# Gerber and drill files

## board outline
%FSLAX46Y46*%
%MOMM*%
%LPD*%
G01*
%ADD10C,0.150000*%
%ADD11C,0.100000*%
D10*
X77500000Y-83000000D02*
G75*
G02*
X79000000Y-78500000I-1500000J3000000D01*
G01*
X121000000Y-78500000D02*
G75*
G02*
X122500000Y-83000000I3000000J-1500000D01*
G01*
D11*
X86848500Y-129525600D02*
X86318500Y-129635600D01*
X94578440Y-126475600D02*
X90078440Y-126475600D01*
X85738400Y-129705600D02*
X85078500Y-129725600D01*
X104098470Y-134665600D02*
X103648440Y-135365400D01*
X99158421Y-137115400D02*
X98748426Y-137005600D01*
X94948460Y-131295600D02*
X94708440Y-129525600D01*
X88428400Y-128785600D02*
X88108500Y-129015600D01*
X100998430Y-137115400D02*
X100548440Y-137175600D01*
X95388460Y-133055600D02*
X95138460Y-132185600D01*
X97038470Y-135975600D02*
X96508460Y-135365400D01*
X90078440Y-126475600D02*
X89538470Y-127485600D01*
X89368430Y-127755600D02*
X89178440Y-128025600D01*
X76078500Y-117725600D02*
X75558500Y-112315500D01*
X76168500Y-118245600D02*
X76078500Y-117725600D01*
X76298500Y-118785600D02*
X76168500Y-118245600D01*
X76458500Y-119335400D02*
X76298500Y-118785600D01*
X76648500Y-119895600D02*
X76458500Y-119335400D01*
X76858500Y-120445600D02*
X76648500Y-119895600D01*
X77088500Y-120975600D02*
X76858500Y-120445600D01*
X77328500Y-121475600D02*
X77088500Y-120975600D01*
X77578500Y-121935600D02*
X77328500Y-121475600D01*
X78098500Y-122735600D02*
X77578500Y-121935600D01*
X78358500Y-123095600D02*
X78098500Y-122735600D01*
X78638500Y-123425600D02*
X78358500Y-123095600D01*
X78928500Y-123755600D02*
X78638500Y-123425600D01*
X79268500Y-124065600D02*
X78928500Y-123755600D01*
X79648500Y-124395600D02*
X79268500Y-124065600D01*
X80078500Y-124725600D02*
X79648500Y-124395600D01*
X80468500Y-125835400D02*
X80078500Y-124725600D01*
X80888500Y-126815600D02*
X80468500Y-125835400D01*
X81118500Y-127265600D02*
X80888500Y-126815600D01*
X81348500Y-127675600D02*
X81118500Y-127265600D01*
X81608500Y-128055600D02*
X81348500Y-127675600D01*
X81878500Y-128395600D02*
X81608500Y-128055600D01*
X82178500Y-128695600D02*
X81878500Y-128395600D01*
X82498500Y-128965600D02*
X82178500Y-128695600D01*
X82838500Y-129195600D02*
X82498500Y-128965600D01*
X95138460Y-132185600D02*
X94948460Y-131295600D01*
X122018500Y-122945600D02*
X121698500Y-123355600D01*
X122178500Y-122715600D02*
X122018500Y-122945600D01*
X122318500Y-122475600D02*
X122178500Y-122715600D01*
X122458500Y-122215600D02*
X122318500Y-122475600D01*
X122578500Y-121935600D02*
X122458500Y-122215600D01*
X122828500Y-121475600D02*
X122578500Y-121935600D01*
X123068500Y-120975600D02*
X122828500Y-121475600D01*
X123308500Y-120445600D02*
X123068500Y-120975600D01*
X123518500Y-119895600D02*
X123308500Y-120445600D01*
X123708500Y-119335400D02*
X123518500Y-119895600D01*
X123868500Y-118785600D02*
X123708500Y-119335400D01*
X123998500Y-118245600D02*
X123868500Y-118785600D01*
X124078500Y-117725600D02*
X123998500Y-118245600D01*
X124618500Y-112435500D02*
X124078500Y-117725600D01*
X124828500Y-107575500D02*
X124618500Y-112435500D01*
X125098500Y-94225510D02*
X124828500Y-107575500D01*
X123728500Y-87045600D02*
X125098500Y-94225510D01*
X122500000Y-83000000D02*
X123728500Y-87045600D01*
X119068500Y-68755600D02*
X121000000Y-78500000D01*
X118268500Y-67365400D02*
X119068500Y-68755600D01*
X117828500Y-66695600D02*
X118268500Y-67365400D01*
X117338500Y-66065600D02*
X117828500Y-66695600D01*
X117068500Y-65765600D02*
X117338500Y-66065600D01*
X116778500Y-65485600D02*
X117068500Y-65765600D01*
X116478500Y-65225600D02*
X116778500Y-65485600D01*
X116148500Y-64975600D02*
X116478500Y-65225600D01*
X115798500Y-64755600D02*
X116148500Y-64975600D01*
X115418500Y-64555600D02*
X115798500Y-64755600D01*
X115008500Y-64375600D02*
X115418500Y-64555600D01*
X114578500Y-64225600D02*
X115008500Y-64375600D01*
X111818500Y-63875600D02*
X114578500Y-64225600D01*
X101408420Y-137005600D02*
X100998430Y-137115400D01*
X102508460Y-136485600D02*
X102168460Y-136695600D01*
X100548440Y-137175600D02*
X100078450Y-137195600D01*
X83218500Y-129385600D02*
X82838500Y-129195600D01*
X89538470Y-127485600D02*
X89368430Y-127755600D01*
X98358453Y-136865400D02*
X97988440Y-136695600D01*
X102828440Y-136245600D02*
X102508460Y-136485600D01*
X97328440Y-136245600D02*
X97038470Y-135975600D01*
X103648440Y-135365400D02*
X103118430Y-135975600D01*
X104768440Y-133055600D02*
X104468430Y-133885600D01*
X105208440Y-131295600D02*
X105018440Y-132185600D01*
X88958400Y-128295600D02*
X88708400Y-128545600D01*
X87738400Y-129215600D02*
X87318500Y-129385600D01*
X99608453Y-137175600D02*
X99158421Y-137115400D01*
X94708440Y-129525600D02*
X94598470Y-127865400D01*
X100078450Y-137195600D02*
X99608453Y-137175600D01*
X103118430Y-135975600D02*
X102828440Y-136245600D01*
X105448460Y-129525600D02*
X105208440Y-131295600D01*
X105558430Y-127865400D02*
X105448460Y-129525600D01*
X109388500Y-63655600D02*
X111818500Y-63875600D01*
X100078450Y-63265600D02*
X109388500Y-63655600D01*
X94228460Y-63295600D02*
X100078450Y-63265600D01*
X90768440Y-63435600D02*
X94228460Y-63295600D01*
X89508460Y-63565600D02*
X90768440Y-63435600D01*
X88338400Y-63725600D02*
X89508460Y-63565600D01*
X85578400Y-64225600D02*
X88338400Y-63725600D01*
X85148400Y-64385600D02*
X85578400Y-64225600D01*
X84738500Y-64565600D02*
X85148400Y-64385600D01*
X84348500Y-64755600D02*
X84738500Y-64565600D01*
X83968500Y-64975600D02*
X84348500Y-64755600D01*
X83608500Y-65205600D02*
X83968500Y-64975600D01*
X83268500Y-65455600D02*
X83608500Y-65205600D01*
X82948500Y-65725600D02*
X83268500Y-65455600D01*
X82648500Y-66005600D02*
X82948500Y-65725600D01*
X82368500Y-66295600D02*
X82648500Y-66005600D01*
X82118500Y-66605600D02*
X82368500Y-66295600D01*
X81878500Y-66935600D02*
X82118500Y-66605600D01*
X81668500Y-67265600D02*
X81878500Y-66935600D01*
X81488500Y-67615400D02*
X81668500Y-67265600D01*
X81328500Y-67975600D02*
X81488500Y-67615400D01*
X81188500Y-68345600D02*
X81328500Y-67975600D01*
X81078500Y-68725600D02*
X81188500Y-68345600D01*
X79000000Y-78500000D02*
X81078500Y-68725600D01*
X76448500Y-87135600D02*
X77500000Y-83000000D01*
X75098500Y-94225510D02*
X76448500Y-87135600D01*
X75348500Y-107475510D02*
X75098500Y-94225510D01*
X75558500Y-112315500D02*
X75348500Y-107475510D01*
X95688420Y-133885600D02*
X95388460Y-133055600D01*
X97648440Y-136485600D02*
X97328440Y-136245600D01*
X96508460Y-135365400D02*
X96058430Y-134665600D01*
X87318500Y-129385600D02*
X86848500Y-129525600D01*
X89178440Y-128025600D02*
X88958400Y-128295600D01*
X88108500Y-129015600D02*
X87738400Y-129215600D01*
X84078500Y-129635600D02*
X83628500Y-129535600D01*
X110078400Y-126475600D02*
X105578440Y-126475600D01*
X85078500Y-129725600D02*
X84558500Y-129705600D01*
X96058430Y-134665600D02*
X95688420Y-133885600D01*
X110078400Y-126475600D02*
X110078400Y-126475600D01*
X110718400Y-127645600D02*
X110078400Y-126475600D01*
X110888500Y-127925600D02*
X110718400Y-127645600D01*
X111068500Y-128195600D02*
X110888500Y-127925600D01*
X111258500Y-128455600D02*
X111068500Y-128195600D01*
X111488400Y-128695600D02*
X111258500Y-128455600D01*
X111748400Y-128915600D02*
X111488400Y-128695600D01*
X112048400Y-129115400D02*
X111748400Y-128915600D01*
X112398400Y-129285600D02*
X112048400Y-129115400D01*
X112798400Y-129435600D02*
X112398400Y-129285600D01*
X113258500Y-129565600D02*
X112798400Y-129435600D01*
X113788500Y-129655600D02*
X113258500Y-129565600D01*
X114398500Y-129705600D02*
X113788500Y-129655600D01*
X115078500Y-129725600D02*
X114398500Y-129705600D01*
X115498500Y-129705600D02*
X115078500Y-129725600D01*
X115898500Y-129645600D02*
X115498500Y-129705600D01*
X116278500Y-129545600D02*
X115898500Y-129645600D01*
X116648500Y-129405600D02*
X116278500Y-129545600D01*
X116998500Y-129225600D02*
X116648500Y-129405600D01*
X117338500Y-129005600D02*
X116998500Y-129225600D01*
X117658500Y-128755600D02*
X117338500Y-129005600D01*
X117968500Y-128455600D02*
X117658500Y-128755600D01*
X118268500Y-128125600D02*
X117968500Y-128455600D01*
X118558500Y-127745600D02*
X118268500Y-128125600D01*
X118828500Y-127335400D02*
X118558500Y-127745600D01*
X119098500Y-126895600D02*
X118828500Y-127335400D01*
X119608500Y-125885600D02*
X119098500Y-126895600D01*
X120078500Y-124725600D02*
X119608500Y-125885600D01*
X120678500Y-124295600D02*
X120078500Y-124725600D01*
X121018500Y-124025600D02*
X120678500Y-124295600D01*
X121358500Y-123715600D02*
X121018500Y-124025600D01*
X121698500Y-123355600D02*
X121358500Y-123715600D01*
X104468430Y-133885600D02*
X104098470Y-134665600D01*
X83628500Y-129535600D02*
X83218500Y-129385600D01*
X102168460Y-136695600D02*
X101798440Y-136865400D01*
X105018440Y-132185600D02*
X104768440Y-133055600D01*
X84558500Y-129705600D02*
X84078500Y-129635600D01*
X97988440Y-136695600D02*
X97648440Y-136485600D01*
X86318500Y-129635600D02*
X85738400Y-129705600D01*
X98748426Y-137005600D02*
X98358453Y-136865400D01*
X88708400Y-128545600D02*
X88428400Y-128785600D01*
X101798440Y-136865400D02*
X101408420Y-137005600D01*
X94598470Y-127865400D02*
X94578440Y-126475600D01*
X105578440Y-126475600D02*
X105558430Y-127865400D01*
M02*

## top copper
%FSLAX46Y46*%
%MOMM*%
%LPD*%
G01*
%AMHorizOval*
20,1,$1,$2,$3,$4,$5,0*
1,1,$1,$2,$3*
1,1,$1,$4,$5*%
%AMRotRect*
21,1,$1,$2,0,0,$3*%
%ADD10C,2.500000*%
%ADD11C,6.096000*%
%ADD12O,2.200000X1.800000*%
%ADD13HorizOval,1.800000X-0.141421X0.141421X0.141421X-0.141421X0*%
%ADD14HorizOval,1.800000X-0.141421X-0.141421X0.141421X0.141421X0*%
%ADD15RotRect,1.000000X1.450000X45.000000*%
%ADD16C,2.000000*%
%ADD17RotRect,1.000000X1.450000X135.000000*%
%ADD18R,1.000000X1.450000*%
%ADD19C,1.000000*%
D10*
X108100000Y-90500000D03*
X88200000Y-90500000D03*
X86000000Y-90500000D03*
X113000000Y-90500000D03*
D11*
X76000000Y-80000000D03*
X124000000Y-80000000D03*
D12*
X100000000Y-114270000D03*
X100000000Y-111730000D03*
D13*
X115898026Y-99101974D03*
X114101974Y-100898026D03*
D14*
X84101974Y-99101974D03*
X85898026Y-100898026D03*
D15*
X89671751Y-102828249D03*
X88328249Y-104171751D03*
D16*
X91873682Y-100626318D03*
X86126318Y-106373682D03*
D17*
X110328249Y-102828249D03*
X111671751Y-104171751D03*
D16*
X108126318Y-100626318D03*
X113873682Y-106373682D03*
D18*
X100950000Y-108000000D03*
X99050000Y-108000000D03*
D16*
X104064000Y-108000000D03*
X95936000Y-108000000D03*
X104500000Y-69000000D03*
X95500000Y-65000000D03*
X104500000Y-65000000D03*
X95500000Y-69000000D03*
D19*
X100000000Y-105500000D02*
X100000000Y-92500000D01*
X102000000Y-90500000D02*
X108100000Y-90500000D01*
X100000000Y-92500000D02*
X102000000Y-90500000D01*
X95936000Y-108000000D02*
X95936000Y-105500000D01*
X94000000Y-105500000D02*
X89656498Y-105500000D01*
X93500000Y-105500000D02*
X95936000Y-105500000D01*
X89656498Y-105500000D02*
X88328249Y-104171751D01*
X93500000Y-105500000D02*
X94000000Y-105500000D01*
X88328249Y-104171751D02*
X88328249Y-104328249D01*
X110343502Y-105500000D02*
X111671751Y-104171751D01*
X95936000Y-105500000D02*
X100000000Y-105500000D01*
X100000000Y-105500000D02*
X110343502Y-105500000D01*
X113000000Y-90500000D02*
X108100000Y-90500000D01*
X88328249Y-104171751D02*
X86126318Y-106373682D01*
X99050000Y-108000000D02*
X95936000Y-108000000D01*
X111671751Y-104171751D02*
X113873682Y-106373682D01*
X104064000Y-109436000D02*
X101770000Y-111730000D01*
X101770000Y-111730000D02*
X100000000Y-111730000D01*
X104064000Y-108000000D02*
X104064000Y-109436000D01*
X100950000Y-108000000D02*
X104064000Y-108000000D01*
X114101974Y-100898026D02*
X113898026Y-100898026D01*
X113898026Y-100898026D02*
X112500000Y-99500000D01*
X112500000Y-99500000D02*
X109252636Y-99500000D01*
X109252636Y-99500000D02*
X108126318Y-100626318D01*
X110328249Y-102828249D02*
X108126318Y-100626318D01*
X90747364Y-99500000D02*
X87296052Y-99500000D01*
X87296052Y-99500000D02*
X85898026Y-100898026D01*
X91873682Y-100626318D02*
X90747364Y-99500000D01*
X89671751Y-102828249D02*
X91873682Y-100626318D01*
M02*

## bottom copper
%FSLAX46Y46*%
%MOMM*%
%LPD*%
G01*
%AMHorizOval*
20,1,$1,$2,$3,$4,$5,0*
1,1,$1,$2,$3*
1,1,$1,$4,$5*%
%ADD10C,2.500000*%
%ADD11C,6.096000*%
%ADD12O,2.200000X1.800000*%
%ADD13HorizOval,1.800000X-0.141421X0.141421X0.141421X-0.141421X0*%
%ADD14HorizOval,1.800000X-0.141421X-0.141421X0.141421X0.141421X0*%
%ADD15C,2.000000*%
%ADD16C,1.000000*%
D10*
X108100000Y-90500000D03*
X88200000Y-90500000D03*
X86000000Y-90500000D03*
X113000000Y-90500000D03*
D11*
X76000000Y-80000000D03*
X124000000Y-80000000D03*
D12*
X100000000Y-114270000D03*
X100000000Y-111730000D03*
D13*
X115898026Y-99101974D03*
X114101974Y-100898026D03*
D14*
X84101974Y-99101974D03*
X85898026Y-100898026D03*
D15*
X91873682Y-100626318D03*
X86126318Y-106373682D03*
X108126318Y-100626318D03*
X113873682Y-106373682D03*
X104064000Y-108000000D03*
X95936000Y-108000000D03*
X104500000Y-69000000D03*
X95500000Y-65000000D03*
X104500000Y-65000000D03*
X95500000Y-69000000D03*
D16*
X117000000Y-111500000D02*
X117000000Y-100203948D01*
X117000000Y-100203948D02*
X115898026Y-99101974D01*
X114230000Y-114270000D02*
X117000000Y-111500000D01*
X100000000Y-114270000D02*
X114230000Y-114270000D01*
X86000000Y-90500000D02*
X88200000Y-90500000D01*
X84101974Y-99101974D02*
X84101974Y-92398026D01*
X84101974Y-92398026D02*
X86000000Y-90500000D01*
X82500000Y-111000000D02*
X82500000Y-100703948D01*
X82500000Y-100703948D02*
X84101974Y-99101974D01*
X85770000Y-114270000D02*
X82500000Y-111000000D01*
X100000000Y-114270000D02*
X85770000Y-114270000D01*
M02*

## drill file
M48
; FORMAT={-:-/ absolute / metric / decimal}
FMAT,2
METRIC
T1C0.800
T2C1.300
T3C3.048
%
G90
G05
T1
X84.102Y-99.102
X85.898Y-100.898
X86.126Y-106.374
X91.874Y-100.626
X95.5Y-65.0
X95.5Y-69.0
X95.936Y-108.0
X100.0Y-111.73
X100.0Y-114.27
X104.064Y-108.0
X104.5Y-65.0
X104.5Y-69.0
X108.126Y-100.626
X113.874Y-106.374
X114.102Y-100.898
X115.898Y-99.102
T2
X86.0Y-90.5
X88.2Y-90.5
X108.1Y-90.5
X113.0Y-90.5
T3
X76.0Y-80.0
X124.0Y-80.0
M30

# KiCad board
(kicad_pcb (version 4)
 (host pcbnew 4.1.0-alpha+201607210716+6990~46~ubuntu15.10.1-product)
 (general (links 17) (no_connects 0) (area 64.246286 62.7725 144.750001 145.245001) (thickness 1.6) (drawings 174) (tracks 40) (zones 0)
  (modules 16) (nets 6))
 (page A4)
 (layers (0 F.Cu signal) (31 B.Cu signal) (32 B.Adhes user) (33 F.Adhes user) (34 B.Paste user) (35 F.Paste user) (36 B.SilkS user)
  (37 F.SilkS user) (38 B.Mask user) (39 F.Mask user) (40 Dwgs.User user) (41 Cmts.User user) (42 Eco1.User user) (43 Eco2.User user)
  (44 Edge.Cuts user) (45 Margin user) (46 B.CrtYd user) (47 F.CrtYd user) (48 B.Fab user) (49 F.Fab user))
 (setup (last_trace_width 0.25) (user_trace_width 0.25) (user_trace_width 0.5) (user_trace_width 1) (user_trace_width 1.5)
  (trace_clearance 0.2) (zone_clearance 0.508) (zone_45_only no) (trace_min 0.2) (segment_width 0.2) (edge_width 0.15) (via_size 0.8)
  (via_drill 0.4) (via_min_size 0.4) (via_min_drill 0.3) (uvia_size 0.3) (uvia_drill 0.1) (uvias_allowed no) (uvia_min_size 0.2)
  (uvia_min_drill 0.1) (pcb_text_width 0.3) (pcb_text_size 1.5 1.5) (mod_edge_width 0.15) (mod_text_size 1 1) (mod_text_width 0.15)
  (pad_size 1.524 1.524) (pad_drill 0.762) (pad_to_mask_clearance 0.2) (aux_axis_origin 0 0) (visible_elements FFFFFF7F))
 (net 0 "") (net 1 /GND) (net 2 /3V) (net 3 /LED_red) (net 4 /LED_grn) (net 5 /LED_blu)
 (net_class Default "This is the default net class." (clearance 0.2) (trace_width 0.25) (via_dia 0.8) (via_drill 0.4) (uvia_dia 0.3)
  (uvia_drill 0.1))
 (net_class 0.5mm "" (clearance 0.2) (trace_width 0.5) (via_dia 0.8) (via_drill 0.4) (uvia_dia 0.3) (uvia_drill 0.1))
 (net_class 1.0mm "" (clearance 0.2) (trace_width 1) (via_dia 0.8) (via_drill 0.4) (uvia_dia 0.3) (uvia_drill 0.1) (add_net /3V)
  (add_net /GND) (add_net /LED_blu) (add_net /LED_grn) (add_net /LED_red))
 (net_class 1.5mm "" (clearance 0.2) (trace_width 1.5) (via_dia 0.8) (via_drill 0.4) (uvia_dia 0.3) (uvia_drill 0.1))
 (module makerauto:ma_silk (layer F.Cu) (at 67.1 109.6)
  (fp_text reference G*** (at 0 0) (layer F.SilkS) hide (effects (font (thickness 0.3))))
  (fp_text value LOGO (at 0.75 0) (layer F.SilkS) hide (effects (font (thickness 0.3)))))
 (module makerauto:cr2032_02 (layer B.Cu) (at 100 90.5 90)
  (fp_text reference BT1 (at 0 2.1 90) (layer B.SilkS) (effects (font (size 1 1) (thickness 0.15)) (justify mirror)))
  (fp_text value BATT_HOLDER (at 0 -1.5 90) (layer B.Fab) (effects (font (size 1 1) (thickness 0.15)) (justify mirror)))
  (pad 2 thru_hole circle (at 0 8.1 90) (size 2.5 2.5) (drill 1.3) (layers *.Cu *.Mask B.SilkS) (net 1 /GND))
  (pad 1 thru_hole circle (at 0 -11.8 90) (size 2.5 2.5) (drill 1.3) (layers *.Cu *.Mask B.SilkS) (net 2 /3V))
  (pad 1 thru_hole circle (at 0 -14 90) (size 2.5 2.5) (drill 1.3) (layers *.Cu *.Mask B.SilkS) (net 2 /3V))
  (pad 2 thru_hole circle (at 0 13 90) (size 2.5 2.5) (drill 1.3) (layers *.Cu *.Mask B.SilkS) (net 1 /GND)))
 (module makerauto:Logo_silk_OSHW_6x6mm (layer B.Cu) (at 100 123 180)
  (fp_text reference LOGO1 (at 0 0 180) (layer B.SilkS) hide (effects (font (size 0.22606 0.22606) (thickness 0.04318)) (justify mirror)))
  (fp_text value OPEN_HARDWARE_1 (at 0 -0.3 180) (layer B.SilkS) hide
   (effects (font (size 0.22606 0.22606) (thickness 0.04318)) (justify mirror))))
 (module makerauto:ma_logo (layer F.Cu) (at 100 100)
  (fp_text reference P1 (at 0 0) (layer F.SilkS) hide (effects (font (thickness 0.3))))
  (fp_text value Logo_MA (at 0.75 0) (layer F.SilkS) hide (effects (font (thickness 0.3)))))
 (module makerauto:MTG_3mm (layer F.Cu) (at 76 80)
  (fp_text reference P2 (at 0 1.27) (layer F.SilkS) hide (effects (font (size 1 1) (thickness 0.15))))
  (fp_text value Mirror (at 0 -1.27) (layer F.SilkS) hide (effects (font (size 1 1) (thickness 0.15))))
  (pad 1 thru_hole circle (at 0 0) (size 6.096 6.096) (drill 3.048) (layers *.Cu *.Mask F.SilkS)))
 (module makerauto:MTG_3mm (layer F.Cu) (at 124 80)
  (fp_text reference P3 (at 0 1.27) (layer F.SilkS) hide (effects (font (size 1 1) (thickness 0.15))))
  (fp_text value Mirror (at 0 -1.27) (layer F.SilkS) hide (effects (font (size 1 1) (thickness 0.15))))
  (pad 1 thru_hole circle (at 0 0) (size 6.096 6.096) (drill 3.048) (layers *.Cu *.Mask F.SilkS)))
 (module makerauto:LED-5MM (layer F.Cu) (at 100 113 90)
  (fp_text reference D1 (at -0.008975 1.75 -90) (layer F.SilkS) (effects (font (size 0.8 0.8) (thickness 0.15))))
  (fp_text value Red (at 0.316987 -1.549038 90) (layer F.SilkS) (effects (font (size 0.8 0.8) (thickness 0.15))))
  (pad 1 thru_hole oval (at -1.27 0 90) (size 1.8 2.2) (drill 0.8) (layers *.Cu *.Mask F.SilkS) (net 2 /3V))
  (pad 2 thru_hole oval (at 1.27 0 90) (size 1.8 2.2) (drill 0.8) (layers *.Cu *.Mask F.SilkS) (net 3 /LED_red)))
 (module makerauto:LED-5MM (layer F.Cu) (at 115 100 225)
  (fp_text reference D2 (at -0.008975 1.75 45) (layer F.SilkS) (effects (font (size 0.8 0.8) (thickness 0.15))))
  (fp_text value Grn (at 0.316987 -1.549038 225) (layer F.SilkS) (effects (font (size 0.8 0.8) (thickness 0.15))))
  (pad 1 thru_hole oval (at -1.27 0 225) (size 1.8 2.2) (drill 0.8) (layers *.Cu *.Mask F.SilkS) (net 2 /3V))
  (pad 2 thru_hole oval (at 1.27 0 225) (size 1.8 2.2) (drill 0.8) (layers *.Cu *.Mask F.SilkS) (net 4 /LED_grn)))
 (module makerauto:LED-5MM (layer F.Cu) (at 85 100 315)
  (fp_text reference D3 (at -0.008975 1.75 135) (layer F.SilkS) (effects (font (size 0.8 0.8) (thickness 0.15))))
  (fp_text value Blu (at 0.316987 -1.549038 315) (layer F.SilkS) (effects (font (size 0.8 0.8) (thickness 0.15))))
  (pad 1 thru_hole oval (at -1.27 0 315) (size 1.8 2.2) (drill 0.8) (layers *.Cu *.Mask F.SilkS) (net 2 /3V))
  (pad 2 thru_hole oval (at 1.27 0 315) (size 1.8 2.2) (drill 0.8) (layers *.Cu *.Mask F.SilkS) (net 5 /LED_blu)))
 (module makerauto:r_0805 (layer F.Cu) (at 89 103.5 45)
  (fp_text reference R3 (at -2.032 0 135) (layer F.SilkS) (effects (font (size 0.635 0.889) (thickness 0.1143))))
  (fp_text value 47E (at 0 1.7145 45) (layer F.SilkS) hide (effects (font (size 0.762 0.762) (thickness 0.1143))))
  (pad 2 smd rect (at 0.95 0 45) (size 1 1.45) (layers F.Cu F.Paste F.Mask) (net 5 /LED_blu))
  (pad 1 smd rect (at -0.95 0 45) (size 1 1.45) (layers F.Cu F.Paste F.Mask) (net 1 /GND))
  (pad 2 thru_hole circle (at 4.064 0 45) (size 2 2) (drill 0.8) (layers *.Cu *.Mask F.SilkS) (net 5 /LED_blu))
  (pad 1 thru_hole circle (at -4.064 0 45) (size 2 2) (drill 0.8) (layers *.Cu *.Mask F.SilkS) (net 1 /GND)))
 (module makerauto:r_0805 (layer F.Cu) (at 111 103.5 135)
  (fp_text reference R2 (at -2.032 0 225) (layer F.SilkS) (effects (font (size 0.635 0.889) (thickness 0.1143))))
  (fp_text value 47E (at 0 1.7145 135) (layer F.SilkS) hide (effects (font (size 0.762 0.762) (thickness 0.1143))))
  (pad 2 smd rect (at 0.95 0 135) (size 1 1.45) (layers F.Cu F.Paste F.Mask) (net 4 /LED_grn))
  (pad 1 smd rect (at -0.95 0 135) (size 1 1.45) (layers F.Cu F.Paste F.Mask) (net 1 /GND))
  (pad 2 thru_hole circle (at 4.064 0 135) (size 2 2) (drill 0.8) (layers *.Cu *.Mask F.SilkS) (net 4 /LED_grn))
  (pad 1 thru_hole circle (at -4.064 0 135) (size 2 2) (drill 0.8) (layers *.Cu *.Mask F.SilkS) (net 1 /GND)))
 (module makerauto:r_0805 (layer F.Cu) (at 100 108)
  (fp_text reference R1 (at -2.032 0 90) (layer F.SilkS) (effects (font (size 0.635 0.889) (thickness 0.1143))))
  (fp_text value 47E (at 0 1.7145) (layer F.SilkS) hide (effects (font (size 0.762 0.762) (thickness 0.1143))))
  (pad 2 smd rect (at 0.95 0) (size 1 1.45) (layers F.Cu F.Paste F.Mask) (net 3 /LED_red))
  (pad 1 smd rect (at -0.95 0) (size 1 1.45) (layers F.Cu F.Paste F.Mask) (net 1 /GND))
  (pad 2 thru_hole circle (at 4.064 0) (size 2 2) (drill 0.8) (layers *.Cu *.Mask F.SilkS) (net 3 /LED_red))
  (pad 1 thru_hole circle (at -4.064 0) (size 2 2) (drill 0.8) (layers *.Cu *.Mask F.SilkS) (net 1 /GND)))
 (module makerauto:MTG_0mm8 (layer F.Cu) (at 104.5 69)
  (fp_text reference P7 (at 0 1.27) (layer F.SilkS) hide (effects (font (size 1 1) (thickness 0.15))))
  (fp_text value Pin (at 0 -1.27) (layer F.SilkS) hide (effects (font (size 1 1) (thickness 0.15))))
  (pad 1 thru_hole circle (at 0 0) (size 2 2) (drill 0.8) (layers *.Cu *.Mask F.SilkS)))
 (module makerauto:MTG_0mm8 (layer F.Cu) (at 95.5 65)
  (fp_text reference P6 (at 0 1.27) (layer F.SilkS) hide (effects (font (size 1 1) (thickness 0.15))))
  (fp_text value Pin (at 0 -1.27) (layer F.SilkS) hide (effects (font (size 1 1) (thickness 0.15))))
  (pad 1 thru_hole circle (at 0 0) (size 2 2) (drill 0.8) (layers *.Cu *.Mask F.SilkS)))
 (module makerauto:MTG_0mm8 (layer F.Cu) (at 104.5 65)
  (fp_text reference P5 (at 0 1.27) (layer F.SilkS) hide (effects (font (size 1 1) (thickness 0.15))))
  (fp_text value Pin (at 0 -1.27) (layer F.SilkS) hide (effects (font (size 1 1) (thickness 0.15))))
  (pad 1 thru_hole circle (at 0 0) (size 2 2) (drill 0.8) (layers *.Cu *.Mask F.SilkS)))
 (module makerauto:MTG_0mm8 (layer F.Cu) (at 95.5 69)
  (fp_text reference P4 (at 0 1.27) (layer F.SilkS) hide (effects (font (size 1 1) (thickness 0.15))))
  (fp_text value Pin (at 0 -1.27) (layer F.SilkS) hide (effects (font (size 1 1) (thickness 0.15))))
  (pad 1 thru_hole circle (at 0 0) (size 2 2) (drill 0.8) (layers *.Cu *.Mask F.SilkS)))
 (gr_arc (start 76 80) (end 77.5 83) (angle 270) (layer Edge.Cuts) (width 0.15))
 (gr_arc (start 124 80) (end 121 78.5) (angle 270) (layer Edge.Cuts) (width 0.15))
 (gr_line (start 86.8485 129.5256) (end 86.3185 129.6356) (layer Edge.Cuts) (width 0.1))
 (gr_line (start 94.57844 126.4756) (end 90.07844 126.4756) (layer Edge.Cuts) (width 0.1))
 (gr_line (start 85.7384 129.7056) (end 85.0785 129.7256) (layer Edge.Cuts) (width 0.1))
 (gr_line (start 104.09847 134.6656) (end 103.64844 135.3654) (layer Edge.Cuts) (width 0.1))
 (gr_line (start 99.158421 137.1154) (end 98.748426 137.0056) (layer Edge.Cuts) (width 0.1))
 (gr_line (start 94.94846 131.2956) (end 94.70844 129.5256) (layer Edge.Cuts) (width 0.1))
 (gr_line (start 88.4284 128.7856) (end 88.1085 129.0156) (layer Edge.Cuts) (width 0.1))
 (gr_line (start 100.99843 137.1154) (end 100.54844 137.1756) (layer Edge.Cuts) (width 0.1))
 (gr_line (start 95.38846 133.0556) (end 95.13846 132.1856) (layer Edge.Cuts) (width 0.1))
 (gr_line (start 97.03847 135.9756) (end 96.50846 135.3654) (layer Edge.Cuts) (width 0.1))
 (gr_line (start 90.07844 126.4756) (end 89.53847 127.4856) (layer Edge.Cuts) (width 0.1))
 (gr_line (start 89.36843 127.7556) (end 89.17844 128.0256) (layer Edge.Cuts) (width 0.1))
 (gr_line (start 76.0785 117.7256) (end 75.5585 112.3155) (layer Edge.Cuts) (width 0.1))
 (gr_line (start 76.1685 118.2456) (end 76.0785 117.7256) (layer Edge.Cuts) (width 0.1))
 (gr_line (start 76.2985 118.7856) (end 76.1685 118.2456) (layer Edge.Cuts) (width 0.1))
 (gr_line (start 76.4585 119.3354) (end 76.2985 118.7856) (layer Edge.Cuts) (width 0.1))
 (gr_line (start 76.6485 119.8956) (end 76.4585 119.3354) (layer Edge.Cuts) (width 0.1))
 (gr_line (start 76.8585 120.4456) (end 76.6485 119.8956) (layer Edge.Cuts) (width 0.1))
 (gr_line (start 77.0885 120.9756) (end 76.8585 120.4456) (layer Edge.Cuts) (width 0.1))
 (gr_line (start 77.3285 121.4756) (end 77.0885 120.9756) (layer Edge.Cuts) (width 0.1))
 (gr_line (start 77.5785 121.9356) (end 77.3285 121.4756) (layer Edge.Cuts) (width 0.1))
 (gr_line (start 78.0985 122.7356) (end 77.5785 121.9356) (layer Edge.Cuts) (width 0.1))
 (gr_line (start 78.3585 123.0956) (end 78.0985 122.7356) (layer Edge.Cuts) (width 0.1))
 (gr_line (start 78.6385 123.4256) (end 78.3585 123.0956) (layer Edge.Cuts) (width 0.1))
 (gr_line (start 78.9285 123.7556) (end 78.6385 123.4256) (layer Edge.Cuts) (width 0.1))
 (gr_line (start 79.2685 124.0656) (end 78.9285 123.7556) (layer Edge.Cuts) (width 0.1))
 (gr_line (start 79.6485 124.3956) (end 79.2685 124.0656) (layer Edge.Cuts) (width 0.1))
 (gr_line (start 80.0785 124.7256) (end 79.6485 124.3956) (layer Edge.Cuts) (width 0.1))
 (gr_line (start 80.4685 125.8354) (end 80.0785 124.7256) (layer Edge.Cuts) (width 0.1))
 (gr_line (start 80.8885 126.8156) (end 80.4685 125.8354) (layer Edge.Cuts) (width 0.1))
 (gr_line (start 81.1185 127.2656) (end 80.8885 126.8156) (layer Edge.Cuts) (width 0.1))
 (gr_line (start 81.3485 127.6756) (end 81.1185 127.2656) (layer Edge.Cuts) (width 0.1))
 (gr_line (start 81.6085 128.0556) (end 81.3485 127.6756) (layer Edge.Cuts) (width 0.1))
 (gr_line (start 81.8785 128.3956) (end 81.6085 128.0556) (layer Edge.Cuts) (width 0.1))
 (gr_line (start 82.1785 128.6956) (end 81.8785 128.3956) (layer Edge.Cuts) (width 0.1))
 (gr_line (start 82.4985 128.9656) (end 82.1785 128.6956) (layer Edge.Cuts) (width 0.1))
 (gr_line (start 82.8385 129.1956) (end 82.4985 128.9656) (layer Edge.Cuts) (width 0.1))
 (gr_line (start 95.13846 132.1856) (end 94.94846 131.2956) (layer Edge.Cuts) (width 0.1))
 (gr_line (start 122.0185 122.9456) (end 121.6985 123.3556) (layer Edge.Cuts) (width 0.1))
 (gr_line (start 122.1785 122.7156) (end 122.0185 122.9456) (layer Edge.Cuts) (width 0.1))
 (gr_line (start 122.3185 122.4756) (end 122.1785 122.7156) (layer Edge.Cuts) (width 0.1))
 (gr_line (start 122.4585 122.2156) (end 122.3185 122.4756) (layer Edge.Cuts) (width 0.1))
 (gr_line (start 122.5785 121.9356) (end 122.4585 122.2156) (layer Edge.Cuts) (width 0.1))
 (gr_line (start 122.8285 121.4756) (end 122.5785 121.9356) (layer Edge.Cuts) (width 0.1))
 (gr_line (start 123.0685 120.9756) (end 122.8285 121.4756) (layer Edge.Cuts) (width 0.1))
 (gr_line (start 123.3085 120.4456) (end 123.0685 120.9756) (layer Edge.Cuts) (width 0.1))
 (gr_line (start 123.5185 119.8956) (end 123.3085 120.4456) (layer Edge.Cuts) (width 0.1))
 (gr_line (start 123.7085 119.3354) (end 123.5185 119.8956) (layer Edge.Cuts) (width 0.1))
 (gr_line (start 123.8685 118.7856) (end 123.7085 119.3354) (layer Edge.Cuts) (width 0.1))
 (gr_line (start 123.9985 118.2456) (end 123.8685 118.7856) (layer Edge.Cuts) (width 0.1))
 (gr_line (start 124.0785 117.7256) (end 123.9985 118.2456) (layer Edge.Cuts) (width 0.1))
 (gr_line (start 124.6185 112.4355) (end 124.0785 117.7256) (layer Edge.Cuts) (width 0.1))
 (gr_line (start 124.8285 107.5755) (end 124.6185 112.4355) (layer Edge.Cuts) (width 0.1))
 (gr_line (start 125.0985 94.22551) (end 124.8285 107.5755) (layer Edge.Cuts) (width 0.1))
 (gr_line (start 123.7285 87.0456) (end 125.0985 94.22551) (layer Edge.Cuts) (width 0.1))
 (gr_line (start 122.5 83) (end 123.7285 87.0456) (layer Edge.Cuts) (width 0.1))
 (gr_line (start 119.0685 68.7556) (end 121 78.5) (layer Edge.Cuts) (width 0.1))
 (gr_line (start 118.2685 67.3654) (end 119.0685 68.7556) (layer Edge.Cuts) (width 0.1))
 (gr_line (start 117.8285 66.6956) (end 118.2685 67.3654) (layer Edge.Cuts) (width 0.1))
 (gr_line (start 117.3385 66.0656) (end 117.8285 66.6956) (layer Edge.Cuts) (width 0.1))
 (gr_line (start 117.0685 65.7656) (end 117.3385 66.0656) (layer Edge.Cuts) (width 0.1))
 (gr_line (start 116.7785 65.4856) (end 117.0685 65.7656) (layer Edge.Cuts) (width 0.1))
 (gr_line (start 116.4785 65.2256) (end 116.7785 65.4856) (layer Edge.Cuts) (width 0.1))
 (gr_line (start 116.1485 64.9756) (end 116.4785 65.2256) (layer Edge.Cuts) (width 0.1))
 (gr_line (start 115.7985 64.7556) (end 116.1485 64.9756) (layer Edge.Cuts) (width 0.1))
 (gr_line (start 115.4185 64.5556) (end 115.7985 64.7556) (layer Edge.Cuts) (width 0.1))
 (gr_line (start 115.0085 64.3756) (end 115.4185 64.5556) (layer Edge.Cuts) (width 0.1))
 (gr_line (start 114.5785 64.2256) (end 115.0085 64.3756) (layer Edge.Cuts) (width 0.1))
 (gr_line (start 111.8185 63.8756) (end 114.5785 64.2256) (layer Edge.Cuts) (width 0.1))
 (gr_line (start 101.40842 137.0056) (end 100.99843 137.1154) (layer Edge.Cuts) (width 0.1))
 (gr_line (start 102.50846 136.4856) (end 102.16846 136.6956) (layer Edge.Cuts) (width 0.1))
 (gr_line (start 100.54844 137.1756) (end 100.07845 137.1956) (layer Edge.Cuts) (width 0.1))
 (gr_line (start 83.2185 129.3856) (end 82.8385 129.1956) (layer Edge.Cuts) (width 0.1))
 (gr_line (start 89.53847 127.4856) (end 89.36843 127.7556) (layer Edge.Cuts) (width 0.1))
 (gr_line (start 98.358453 136.8654) (end 97.98844 136.6956) (layer Edge.Cuts) (width 0.1))
 (gr_line (start 102.82844 136.2456) (end 102.50846 136.4856) (layer Edge.Cuts) (width 0.1))
 (gr_line (start 97.32844 136.2456) (end 97.03847 135.9756) (layer Edge.Cuts) (width 0.1))
 (gr_line (start 103.64844 135.3654) (end 103.11843 135.9756) (layer Edge.Cuts) (width 0.1))
 (gr_line (start 104.76844 133.0556) (end 104.46843 133.8856) (layer Edge.Cuts) (width 0.1))
 (gr_line (start 105.20844 131.2956) (end 105.01844 132.1856) (layer Edge.Cuts) (width 0.1))
 (gr_line (start 88.9584 128.2956) (end 88.7084 128.5456) (layer Edge.Cuts) (width 0.1))
 (gr_line (start 87.7384 129.2156) (end 87.3185 129.3856) (layer Edge.Cuts) (width 0.1))
 (gr_line (start 99.608453 137.1756) (end 99.158421 137.1154) (layer Edge.Cuts) (width 0.1))
 (gr_line (start 94.70844 129.5256) (end 94.59847 127.8654) (layer Edge.Cuts) (width 0.1))
 (gr_line (start 100.07845 137.1956) (end 99.608453 137.1756) (layer Edge.Cuts) (width 0.1))
 (gr_line (start 103.11843 135.9756) (end 102.82844 136.2456) (layer Edge.Cuts) (width 0.1))
 (gr_line (start 105.44846 129.5256) (end 105.20844 131.2956) (layer Edge.Cuts) (width 0.1))
 (gr_line (start 105.55843 127.8654) (end 105.44846 129.5256) (layer Edge.Cuts) (width 0.1))
 (gr_line (start 109.3885 63.6556) (end 111.8185 63.8756) (layer Edge.Cuts) (width 0.1))
 (gr_line (start 100.07845 63.2656) (end 109.3885 63.6556) (layer Edge.Cuts) (width 0.1))
 (gr_line (start 94.22846 63.2956) (end 100.07845 63.2656) (layer Edge.Cuts) (width 0.1))
 (gr_line (start 90.76844 63.4356) (end 94.22846 63.2956) (layer Edge.Cuts) (width 0.1))
 (gr_line (start 89.50846 63.5656) (end 90.76844 63.4356) (layer Edge.Cuts) (width 0.1))
 (gr_line (start 88.3384 63.7256) (end 89.50846 63.5656) (layer Edge.Cuts) (width 0.1))
 (gr_line (start 85.5784 64.2256) (end 88.3384 63.7256) (layer Edge.Cuts) (width 0.1))
 (gr_line (start 85.1484 64.3856) (end 85.5784 64.2256) (layer Edge.Cuts) (width 0.1))
 (gr_line (start 84.7385 64.5656) (end 85.1484 64.3856) (layer Edge.Cuts) (width 0.1))
 (gr_line (start 84.3485 64.7556) (end 84.7385 64.5656) (layer Edge.Cuts) (width 0.1))
 (gr_line (start 83.9685 64.9756) (end 84.3485 64.7556) (layer Edge.Cuts) (width 0.1))
 (gr_line (start 83.6085 65.2056) (end 83.9685 64.9756) (layer Edge.Cuts) (width 0.1))
 (gr_line (start 83.2685 65.4556) (end 83.6085 65.2056) (layer Edge.Cuts) (width 0.1))
 (gr_line (start 82.9485 65.7256) (end 83.2685 65.4556) (layer Edge.Cuts) (width 0.1))
 (gr_line (start 82.6485 66.0056) (end 82.9485 65.7256) (layer Edge.Cuts) (width 0.1))
 (gr_line (start 82.3685 66.2956) (end 82.6485 66.0056) (layer Edge.Cuts) (width 0.1))
 (gr_line (start 82.1185 66.6056) (end 82.3685 66.2956) (layer Edge.Cuts) (width 0.1))
 (gr_line (start 81.8785 66.9356) (end 82.1185 66.6056) (layer Edge.Cuts) (width 0.1))
 (gr_line (start 81.6685 67.2656) (end 81.8785 66.9356) (layer Edge.Cuts) (width 0.1))
 (gr_line (start 81.4885 67.6154) (end 81.6685 67.2656) (layer Edge.Cuts) (width 0.1))
 (gr_line (start 81.3285 67.9756) (end 81.4885 67.6154) (layer Edge.Cuts) (width 0.1))
 (gr_line (start 81.1885 68.3456) (end 81.3285 67.9756) (layer Edge.Cuts) (width 0.1))
 (gr_line (start 81.0785 68.7256) (end 81.1885 68.3456) (layer Edge.Cuts) (width 0.1))
 (gr_line (start 79 78.5) (end 81.0785 68.7256) (layer Edge.Cuts) (width 0.1))
 (gr_line (start 76.4485 87.1356) (end 77.5 83) (layer Edge.Cuts) (width 0.1))
 (gr_line (start 75.0985 94.22551) (end 76.4485 87.1356) (layer Edge.Cuts) (width 0.1))
 (gr_line (start 75.3485 107.47551) (end 75.0985 94.22551) (layer Edge.Cuts) (width 0.1))
 (gr_line (start 75.5585 112.3155) (end 75.3485 107.47551) (layer Edge.Cuts) (width 0.1))
 (gr_line (start 95.68842 133.8856) (end 95.38846 133.0556) (layer Edge.Cuts) (width 0.1))
 (gr_line (start 97.64844 136.4856) (end 97.32844 136.2456) (layer Edge.Cuts) (width 0.1))
 (gr_line (start 96.50846 135.3654) (end 96.05843 134.6656) (layer Edge.Cuts) (width 0.1))
 (gr_line (start 87.3185 129.3856) (end 86.8485 129.5256) (layer Edge.Cuts) (width 0.1))
 (gr_line (start 89.17844 128.0256) (end 88.9584 128.2956) (layer Edge.Cuts) (width 0.1))
 (gr_line (start 88.1085 129.0156) (end 87.7384 129.2156) (layer Edge.Cuts) (width 0.1))
 (gr_line (start 84.0785 129.6356) (end 83.6285 129.5356) (layer Edge.Cuts) (width 0.1))
 (gr_line (start 110.0784 126.4756) (end 105.57844 126.4756) (layer Edge.Cuts) (width 0.1))
 (gr_line (start 85.0785 129.7256) (end 84.5585 129.7056) (layer Edge.Cuts) (width 0.1))
 (gr_line (start 96.05843 134.6656) (end 95.68842 133.8856) (layer Edge.Cuts) (width 0.1))
 (gr_line (start 110.0784 126.4756) (end 110.0784 126.4756) (layer Edge.Cuts) (width 0.1))
 (gr_line (start 110.7184 127.6456) (end 110.0784 126.4756) (layer Edge.Cuts) (width 0.1))
 (gr_line (start 110.8885 127.9256) (end 110.7184 127.6456) (layer Edge.Cuts) (width 0.1))
 (gr_line (start 111.0685 128.1956) (end 110.8885 127.9256) (layer Edge.Cuts) (width 0.1))
 (gr_line (start 111.2585 128.4556) (end 111.0685 128.1956) (layer Edge.Cuts) (width 0.1))
 (gr_line (start 111.4884 128.6956) (end 111.2585 128.4556) (layer Edge.Cuts) (width 0.1))
 (gr_line (start 111.7484 128.9156) (end 111.4884 128.6956) (layer Edge.Cuts) (width 0.1))
 (gr_line (start 112.0484 129.1154) (end 111.7484 128.9156) (layer Edge.Cuts) (width 0.1))
 (gr_line (start 112.3984 129.2856) (end 112.0484 129.1154) (layer Edge.Cuts) (width 0.1))
 (gr_line (start 112.7984 129.4356) (end 112.3984 129.2856) (layer Edge.Cuts) (width 0.1))
 (gr_line (start 113.2585 129.5656) (end 112.7984 129.4356) (layer Edge.Cuts) (width 0.1))
 (gr_line (start 113.7885 129.6556) (end 113.2585 129.5656) (layer Edge.Cuts) (width 0.1))
 (gr_line (start 114.3985 129.7056) (end 113.7885 129.6556) (layer Edge.Cuts) (width 0.1))
 (gr_line (start 115.0785 129.7256) (end 114.3985 129.7056) (layer Edge.Cuts) (width 0.1))
 (gr_line (start 115.4985 129.7056) (end 115.0785 129.7256) (layer Edge.Cuts) (width 0.1))
 (gr_line (start 115.8985 129.6456) (end 115.4985 129.7056) (layer Edge.Cuts) (width 0.1))
 (gr_line (start 116.2785 129.5456) (end 115.8985 129.6456) (layer Edge.Cuts) (width 0.1))
 (gr_line (start 116.6485 129.4056) (end 116.2785 129.5456) (layer Edge.Cuts) (width 0.1))
 (gr_line (start 116.9985 129.2256) (end 116.6485 129.4056) (layer Edge.Cuts) (width 0.1))
 (gr_line (start 117.3385 129.0056) (end 116.9985 129.2256) (layer Edge.Cuts) (width 0.1))
 (gr_line (start 117.6585 128.7556) (end 117.3385 129.0056) (layer Edge.Cuts) (width 0.1))
 (gr_line (start 117.9685 128.4556) (end 117.6585 128.7556) (layer Edge.Cuts) (width 0.1))
 (gr_line (start 118.2685 128.1256) (end 117.9685 128.4556) (layer Edge.Cuts) (width 0.1))
 (gr_line (start 118.5585 127.7456) (end 118.2685 128.1256) (layer Edge.Cuts) (width 0.1))
 (gr_line (start 118.8285 127.3354) (end 118.5585 127.7456) (layer Edge.Cuts) (width 0.1))
 (gr_line (start 119.0985 126.8956) (end 118.8285 127.3354) (layer Edge.Cuts) (width 0.1))
 (gr_line (start 119.6085 125.8856) (end 119.0985 126.8956) (layer Edge.Cuts) (width 0.1))
 (gr_line (start 120.0785 124.7256) (end 119.6085 125.8856) (layer Edge.Cuts) (width 0.1))
 (gr_line (start 120.6785 124.2956) (end 120.0785 124.7256) (layer Edge.Cuts) (width 0.1))
 (gr_line (start 121.0185 124.0256) (end 120.6785 124.2956) (layer Edge.Cuts) (width 0.1))
 (gr_line (start 121.3585 123.7156) (end 121.0185 124.0256) (layer Edge.Cuts) (width 0.1))
 (gr_line (start 121.6985 123.3556) (end 121.3585 123.7156) (layer Edge.Cuts) (width 0.1))
 (gr_line (start 104.46843 133.8856) (end 104.09847 134.6656) (layer Edge.Cuts) (width 0.1))
 (gr_line (start 83.6285 129.5356) (end 83.2185 129.3856) (layer Edge.Cuts) (width 0.1))
 (gr_line (start 102.16846 136.6956) (end 101.79844 136.8654) (layer Edge.Cuts) (width 0.1))
 (gr_line (start 105.01844 132.1856) (end 104.76844 133.0556) (layer Edge.Cuts) (width 0.1))
 (gr_line (start 84.5585 129.7056) (end 84.0785 129.6356) (layer Edge.Cuts) (width 0.1))
 (gr_line (start 97.98844 136.6956) (end 97.64844 136.4856) (layer Edge.Cuts) (width 0.1))
 (gr_line (start 86.3185 129.6356) (end 85.7384 129.7056) (layer Edge.Cuts) (width 0.1))
 (gr_line (start 98.748426 137.0056) (end 98.358453 136.8654) (layer Edge.Cuts) (width 0.1))
 (gr_line (start 88.7084 128.5456) (end 88.4284 128.7856) (layer Edge.Cuts) (width 0.1))
 (gr_line (start 101.79844 136.8654) (end 101.40842 137.0056) (layer Edge.Cuts) (width 0.1))
 (gr_line (start 94.59847 127.8654) (end 94.57844 126.4756) (layer Edge.Cuts) (width 0.1))
 (gr_line (start 105.57844 126.4756) (end 105.55843 127.8654) (layer Edge.Cuts) (width 0.1))
 (segment (start 100 105.5) (end 100 92.5) (width 1) (layer F.Cu) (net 1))
 (segment (start 102 90.5) (end 108.1 90.5) (width 1) (layer F.Cu) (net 1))
 (segment (start 100 92.5) (end 102 90.5) (width 1) (layer F.Cu) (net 1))
 (segment (start 95.936 108) (end 95.936 105.5) (width 1) (layer F.Cu) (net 1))
 (segment (start 94 105.5) (end 89.656498 105.5) (width 1) (layer F.Cu) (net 1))
 (segment (start 93.5 105.5) (end 95.936 105.5) (width 1) (layer F.Cu) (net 1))
 (segment (start 89.656498 105.5) (end 88.328249 104.171751) (width 1) (layer F.Cu) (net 1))
 (segment (start 93.5 105.5) (end 94 105.5) (width 1) (layer F.Cu) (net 1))
 (segment (start 88.328249 104.171751) (end 88.328249 104.328249) (width 1) (layer F.Cu) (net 1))
 (segment (start 110.343502 105.5) (end 111.671751 104.171751) (width 1) (layer F.Cu) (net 1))
 (segment (start 95.936 105.5) (end 100 105.5) (width 1) (layer F.Cu) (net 1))
 (segment (start 100 105.5) (end 110.343502 105.5) (width 1) (layer F.Cu) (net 1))
 (segment (start 113 90.5) (end 108.1 90.5) (width 1) (layer F.Cu) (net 1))
 (segment (start 88.328249 104.171751) (end 86.126318 106.373682) (width 1) (layer F.Cu) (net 1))
 (segment (start 99.05 108) (end 95.936 108) (width 1) (layer F.Cu) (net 1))
 (segment (start 111.671751 104.171751) (end 113.873682 106.373682) (width 1) (layer F.Cu) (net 1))
 (segment (start 117 111.5) (end 117 100.203948) (width 1) (layer B.Cu) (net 2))
 (segment (start 117 100.203948) (end 115.898026 99.101974) (width 1) (layer B.Cu) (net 2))
 (segment (start 114.23 114.27) (end 117 111.5) (width 1) (layer B.Cu) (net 2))
 (segment (start 100 114.27) (end 114.23 114.27) (width 1) (layer B.Cu) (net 2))
 (segment (start 86 90.5) (end 88.2 90.5) (width 1) (layer B.Cu) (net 2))
 (segment (start 84.101974 99.101974) (end 84.101974 92.398026) (width 1) (layer B.Cu) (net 2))
 (segment (start 84.101974 92.398026) (end 86 90.5) (width 1) (layer B.Cu) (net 2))
 (segment (start 82.5 111) (end 82.5 100.703948) (width 1) (layer B.Cu) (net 2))
 (segment (start 82.5 100.703948) (end 84.101974 99.101974) (width 1) (layer B.Cu) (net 2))
 (segment (start 85.77 114.27) (end 82.5 111) (width 1) (layer B.Cu) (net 2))
 (segment (start 100 114.27) (end 85.77 114.27) (width 1) (layer B.Cu) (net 2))
 (segment (start 104.064 109.436) (end 101.77 111.73) (width 1) (layer F.Cu) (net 3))
 (segment (start 101.77 111.73) (end 100 111.73) (width 1) (layer F.Cu) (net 3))
 (segment (start 104.064 108) (end 104.064 109.436) (width 1) (layer F.Cu) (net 3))
 (segment (start 100.95 108) (end 104.064 108) (width 1) (layer F.Cu) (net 3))
 (segment (start 114.101974 100.898026) (end 113.898026 100.898026) (width 1) (layer F.Cu) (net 4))
 (segment (start 113.898026 100.898026) (end 112.5 99.5) (width 1) (layer F.Cu) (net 4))
 (segment (start 112.5 99.5) (end 109.252636 99.5) (width 1) (layer F.Cu) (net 4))
 (segment (start 109.252636 99.5) (end 108.126318 100.626318) (width 1) (layer F.Cu) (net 4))
 (segment (start 110.328249 102.828249) (end 108.126318 100.626318) (width 1) (layer F.Cu) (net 4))
 (segment (start 90.747364 99.5) (end 87.296052 99.5) (width 1) (layer F.Cu) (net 5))
 (segment (start 87.296052 99.5) (end 85.898026 100.898026) (width 1) (layer F.Cu) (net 5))
 (segment (start 91.873682 100.626318) (end 90.747364 99.5) (width 1) (layer F.Cu) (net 5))
 (segment (start 89.671751 102.828249) (end 91.873682 100.626318) (width 1) (layer F.Cu) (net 5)))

